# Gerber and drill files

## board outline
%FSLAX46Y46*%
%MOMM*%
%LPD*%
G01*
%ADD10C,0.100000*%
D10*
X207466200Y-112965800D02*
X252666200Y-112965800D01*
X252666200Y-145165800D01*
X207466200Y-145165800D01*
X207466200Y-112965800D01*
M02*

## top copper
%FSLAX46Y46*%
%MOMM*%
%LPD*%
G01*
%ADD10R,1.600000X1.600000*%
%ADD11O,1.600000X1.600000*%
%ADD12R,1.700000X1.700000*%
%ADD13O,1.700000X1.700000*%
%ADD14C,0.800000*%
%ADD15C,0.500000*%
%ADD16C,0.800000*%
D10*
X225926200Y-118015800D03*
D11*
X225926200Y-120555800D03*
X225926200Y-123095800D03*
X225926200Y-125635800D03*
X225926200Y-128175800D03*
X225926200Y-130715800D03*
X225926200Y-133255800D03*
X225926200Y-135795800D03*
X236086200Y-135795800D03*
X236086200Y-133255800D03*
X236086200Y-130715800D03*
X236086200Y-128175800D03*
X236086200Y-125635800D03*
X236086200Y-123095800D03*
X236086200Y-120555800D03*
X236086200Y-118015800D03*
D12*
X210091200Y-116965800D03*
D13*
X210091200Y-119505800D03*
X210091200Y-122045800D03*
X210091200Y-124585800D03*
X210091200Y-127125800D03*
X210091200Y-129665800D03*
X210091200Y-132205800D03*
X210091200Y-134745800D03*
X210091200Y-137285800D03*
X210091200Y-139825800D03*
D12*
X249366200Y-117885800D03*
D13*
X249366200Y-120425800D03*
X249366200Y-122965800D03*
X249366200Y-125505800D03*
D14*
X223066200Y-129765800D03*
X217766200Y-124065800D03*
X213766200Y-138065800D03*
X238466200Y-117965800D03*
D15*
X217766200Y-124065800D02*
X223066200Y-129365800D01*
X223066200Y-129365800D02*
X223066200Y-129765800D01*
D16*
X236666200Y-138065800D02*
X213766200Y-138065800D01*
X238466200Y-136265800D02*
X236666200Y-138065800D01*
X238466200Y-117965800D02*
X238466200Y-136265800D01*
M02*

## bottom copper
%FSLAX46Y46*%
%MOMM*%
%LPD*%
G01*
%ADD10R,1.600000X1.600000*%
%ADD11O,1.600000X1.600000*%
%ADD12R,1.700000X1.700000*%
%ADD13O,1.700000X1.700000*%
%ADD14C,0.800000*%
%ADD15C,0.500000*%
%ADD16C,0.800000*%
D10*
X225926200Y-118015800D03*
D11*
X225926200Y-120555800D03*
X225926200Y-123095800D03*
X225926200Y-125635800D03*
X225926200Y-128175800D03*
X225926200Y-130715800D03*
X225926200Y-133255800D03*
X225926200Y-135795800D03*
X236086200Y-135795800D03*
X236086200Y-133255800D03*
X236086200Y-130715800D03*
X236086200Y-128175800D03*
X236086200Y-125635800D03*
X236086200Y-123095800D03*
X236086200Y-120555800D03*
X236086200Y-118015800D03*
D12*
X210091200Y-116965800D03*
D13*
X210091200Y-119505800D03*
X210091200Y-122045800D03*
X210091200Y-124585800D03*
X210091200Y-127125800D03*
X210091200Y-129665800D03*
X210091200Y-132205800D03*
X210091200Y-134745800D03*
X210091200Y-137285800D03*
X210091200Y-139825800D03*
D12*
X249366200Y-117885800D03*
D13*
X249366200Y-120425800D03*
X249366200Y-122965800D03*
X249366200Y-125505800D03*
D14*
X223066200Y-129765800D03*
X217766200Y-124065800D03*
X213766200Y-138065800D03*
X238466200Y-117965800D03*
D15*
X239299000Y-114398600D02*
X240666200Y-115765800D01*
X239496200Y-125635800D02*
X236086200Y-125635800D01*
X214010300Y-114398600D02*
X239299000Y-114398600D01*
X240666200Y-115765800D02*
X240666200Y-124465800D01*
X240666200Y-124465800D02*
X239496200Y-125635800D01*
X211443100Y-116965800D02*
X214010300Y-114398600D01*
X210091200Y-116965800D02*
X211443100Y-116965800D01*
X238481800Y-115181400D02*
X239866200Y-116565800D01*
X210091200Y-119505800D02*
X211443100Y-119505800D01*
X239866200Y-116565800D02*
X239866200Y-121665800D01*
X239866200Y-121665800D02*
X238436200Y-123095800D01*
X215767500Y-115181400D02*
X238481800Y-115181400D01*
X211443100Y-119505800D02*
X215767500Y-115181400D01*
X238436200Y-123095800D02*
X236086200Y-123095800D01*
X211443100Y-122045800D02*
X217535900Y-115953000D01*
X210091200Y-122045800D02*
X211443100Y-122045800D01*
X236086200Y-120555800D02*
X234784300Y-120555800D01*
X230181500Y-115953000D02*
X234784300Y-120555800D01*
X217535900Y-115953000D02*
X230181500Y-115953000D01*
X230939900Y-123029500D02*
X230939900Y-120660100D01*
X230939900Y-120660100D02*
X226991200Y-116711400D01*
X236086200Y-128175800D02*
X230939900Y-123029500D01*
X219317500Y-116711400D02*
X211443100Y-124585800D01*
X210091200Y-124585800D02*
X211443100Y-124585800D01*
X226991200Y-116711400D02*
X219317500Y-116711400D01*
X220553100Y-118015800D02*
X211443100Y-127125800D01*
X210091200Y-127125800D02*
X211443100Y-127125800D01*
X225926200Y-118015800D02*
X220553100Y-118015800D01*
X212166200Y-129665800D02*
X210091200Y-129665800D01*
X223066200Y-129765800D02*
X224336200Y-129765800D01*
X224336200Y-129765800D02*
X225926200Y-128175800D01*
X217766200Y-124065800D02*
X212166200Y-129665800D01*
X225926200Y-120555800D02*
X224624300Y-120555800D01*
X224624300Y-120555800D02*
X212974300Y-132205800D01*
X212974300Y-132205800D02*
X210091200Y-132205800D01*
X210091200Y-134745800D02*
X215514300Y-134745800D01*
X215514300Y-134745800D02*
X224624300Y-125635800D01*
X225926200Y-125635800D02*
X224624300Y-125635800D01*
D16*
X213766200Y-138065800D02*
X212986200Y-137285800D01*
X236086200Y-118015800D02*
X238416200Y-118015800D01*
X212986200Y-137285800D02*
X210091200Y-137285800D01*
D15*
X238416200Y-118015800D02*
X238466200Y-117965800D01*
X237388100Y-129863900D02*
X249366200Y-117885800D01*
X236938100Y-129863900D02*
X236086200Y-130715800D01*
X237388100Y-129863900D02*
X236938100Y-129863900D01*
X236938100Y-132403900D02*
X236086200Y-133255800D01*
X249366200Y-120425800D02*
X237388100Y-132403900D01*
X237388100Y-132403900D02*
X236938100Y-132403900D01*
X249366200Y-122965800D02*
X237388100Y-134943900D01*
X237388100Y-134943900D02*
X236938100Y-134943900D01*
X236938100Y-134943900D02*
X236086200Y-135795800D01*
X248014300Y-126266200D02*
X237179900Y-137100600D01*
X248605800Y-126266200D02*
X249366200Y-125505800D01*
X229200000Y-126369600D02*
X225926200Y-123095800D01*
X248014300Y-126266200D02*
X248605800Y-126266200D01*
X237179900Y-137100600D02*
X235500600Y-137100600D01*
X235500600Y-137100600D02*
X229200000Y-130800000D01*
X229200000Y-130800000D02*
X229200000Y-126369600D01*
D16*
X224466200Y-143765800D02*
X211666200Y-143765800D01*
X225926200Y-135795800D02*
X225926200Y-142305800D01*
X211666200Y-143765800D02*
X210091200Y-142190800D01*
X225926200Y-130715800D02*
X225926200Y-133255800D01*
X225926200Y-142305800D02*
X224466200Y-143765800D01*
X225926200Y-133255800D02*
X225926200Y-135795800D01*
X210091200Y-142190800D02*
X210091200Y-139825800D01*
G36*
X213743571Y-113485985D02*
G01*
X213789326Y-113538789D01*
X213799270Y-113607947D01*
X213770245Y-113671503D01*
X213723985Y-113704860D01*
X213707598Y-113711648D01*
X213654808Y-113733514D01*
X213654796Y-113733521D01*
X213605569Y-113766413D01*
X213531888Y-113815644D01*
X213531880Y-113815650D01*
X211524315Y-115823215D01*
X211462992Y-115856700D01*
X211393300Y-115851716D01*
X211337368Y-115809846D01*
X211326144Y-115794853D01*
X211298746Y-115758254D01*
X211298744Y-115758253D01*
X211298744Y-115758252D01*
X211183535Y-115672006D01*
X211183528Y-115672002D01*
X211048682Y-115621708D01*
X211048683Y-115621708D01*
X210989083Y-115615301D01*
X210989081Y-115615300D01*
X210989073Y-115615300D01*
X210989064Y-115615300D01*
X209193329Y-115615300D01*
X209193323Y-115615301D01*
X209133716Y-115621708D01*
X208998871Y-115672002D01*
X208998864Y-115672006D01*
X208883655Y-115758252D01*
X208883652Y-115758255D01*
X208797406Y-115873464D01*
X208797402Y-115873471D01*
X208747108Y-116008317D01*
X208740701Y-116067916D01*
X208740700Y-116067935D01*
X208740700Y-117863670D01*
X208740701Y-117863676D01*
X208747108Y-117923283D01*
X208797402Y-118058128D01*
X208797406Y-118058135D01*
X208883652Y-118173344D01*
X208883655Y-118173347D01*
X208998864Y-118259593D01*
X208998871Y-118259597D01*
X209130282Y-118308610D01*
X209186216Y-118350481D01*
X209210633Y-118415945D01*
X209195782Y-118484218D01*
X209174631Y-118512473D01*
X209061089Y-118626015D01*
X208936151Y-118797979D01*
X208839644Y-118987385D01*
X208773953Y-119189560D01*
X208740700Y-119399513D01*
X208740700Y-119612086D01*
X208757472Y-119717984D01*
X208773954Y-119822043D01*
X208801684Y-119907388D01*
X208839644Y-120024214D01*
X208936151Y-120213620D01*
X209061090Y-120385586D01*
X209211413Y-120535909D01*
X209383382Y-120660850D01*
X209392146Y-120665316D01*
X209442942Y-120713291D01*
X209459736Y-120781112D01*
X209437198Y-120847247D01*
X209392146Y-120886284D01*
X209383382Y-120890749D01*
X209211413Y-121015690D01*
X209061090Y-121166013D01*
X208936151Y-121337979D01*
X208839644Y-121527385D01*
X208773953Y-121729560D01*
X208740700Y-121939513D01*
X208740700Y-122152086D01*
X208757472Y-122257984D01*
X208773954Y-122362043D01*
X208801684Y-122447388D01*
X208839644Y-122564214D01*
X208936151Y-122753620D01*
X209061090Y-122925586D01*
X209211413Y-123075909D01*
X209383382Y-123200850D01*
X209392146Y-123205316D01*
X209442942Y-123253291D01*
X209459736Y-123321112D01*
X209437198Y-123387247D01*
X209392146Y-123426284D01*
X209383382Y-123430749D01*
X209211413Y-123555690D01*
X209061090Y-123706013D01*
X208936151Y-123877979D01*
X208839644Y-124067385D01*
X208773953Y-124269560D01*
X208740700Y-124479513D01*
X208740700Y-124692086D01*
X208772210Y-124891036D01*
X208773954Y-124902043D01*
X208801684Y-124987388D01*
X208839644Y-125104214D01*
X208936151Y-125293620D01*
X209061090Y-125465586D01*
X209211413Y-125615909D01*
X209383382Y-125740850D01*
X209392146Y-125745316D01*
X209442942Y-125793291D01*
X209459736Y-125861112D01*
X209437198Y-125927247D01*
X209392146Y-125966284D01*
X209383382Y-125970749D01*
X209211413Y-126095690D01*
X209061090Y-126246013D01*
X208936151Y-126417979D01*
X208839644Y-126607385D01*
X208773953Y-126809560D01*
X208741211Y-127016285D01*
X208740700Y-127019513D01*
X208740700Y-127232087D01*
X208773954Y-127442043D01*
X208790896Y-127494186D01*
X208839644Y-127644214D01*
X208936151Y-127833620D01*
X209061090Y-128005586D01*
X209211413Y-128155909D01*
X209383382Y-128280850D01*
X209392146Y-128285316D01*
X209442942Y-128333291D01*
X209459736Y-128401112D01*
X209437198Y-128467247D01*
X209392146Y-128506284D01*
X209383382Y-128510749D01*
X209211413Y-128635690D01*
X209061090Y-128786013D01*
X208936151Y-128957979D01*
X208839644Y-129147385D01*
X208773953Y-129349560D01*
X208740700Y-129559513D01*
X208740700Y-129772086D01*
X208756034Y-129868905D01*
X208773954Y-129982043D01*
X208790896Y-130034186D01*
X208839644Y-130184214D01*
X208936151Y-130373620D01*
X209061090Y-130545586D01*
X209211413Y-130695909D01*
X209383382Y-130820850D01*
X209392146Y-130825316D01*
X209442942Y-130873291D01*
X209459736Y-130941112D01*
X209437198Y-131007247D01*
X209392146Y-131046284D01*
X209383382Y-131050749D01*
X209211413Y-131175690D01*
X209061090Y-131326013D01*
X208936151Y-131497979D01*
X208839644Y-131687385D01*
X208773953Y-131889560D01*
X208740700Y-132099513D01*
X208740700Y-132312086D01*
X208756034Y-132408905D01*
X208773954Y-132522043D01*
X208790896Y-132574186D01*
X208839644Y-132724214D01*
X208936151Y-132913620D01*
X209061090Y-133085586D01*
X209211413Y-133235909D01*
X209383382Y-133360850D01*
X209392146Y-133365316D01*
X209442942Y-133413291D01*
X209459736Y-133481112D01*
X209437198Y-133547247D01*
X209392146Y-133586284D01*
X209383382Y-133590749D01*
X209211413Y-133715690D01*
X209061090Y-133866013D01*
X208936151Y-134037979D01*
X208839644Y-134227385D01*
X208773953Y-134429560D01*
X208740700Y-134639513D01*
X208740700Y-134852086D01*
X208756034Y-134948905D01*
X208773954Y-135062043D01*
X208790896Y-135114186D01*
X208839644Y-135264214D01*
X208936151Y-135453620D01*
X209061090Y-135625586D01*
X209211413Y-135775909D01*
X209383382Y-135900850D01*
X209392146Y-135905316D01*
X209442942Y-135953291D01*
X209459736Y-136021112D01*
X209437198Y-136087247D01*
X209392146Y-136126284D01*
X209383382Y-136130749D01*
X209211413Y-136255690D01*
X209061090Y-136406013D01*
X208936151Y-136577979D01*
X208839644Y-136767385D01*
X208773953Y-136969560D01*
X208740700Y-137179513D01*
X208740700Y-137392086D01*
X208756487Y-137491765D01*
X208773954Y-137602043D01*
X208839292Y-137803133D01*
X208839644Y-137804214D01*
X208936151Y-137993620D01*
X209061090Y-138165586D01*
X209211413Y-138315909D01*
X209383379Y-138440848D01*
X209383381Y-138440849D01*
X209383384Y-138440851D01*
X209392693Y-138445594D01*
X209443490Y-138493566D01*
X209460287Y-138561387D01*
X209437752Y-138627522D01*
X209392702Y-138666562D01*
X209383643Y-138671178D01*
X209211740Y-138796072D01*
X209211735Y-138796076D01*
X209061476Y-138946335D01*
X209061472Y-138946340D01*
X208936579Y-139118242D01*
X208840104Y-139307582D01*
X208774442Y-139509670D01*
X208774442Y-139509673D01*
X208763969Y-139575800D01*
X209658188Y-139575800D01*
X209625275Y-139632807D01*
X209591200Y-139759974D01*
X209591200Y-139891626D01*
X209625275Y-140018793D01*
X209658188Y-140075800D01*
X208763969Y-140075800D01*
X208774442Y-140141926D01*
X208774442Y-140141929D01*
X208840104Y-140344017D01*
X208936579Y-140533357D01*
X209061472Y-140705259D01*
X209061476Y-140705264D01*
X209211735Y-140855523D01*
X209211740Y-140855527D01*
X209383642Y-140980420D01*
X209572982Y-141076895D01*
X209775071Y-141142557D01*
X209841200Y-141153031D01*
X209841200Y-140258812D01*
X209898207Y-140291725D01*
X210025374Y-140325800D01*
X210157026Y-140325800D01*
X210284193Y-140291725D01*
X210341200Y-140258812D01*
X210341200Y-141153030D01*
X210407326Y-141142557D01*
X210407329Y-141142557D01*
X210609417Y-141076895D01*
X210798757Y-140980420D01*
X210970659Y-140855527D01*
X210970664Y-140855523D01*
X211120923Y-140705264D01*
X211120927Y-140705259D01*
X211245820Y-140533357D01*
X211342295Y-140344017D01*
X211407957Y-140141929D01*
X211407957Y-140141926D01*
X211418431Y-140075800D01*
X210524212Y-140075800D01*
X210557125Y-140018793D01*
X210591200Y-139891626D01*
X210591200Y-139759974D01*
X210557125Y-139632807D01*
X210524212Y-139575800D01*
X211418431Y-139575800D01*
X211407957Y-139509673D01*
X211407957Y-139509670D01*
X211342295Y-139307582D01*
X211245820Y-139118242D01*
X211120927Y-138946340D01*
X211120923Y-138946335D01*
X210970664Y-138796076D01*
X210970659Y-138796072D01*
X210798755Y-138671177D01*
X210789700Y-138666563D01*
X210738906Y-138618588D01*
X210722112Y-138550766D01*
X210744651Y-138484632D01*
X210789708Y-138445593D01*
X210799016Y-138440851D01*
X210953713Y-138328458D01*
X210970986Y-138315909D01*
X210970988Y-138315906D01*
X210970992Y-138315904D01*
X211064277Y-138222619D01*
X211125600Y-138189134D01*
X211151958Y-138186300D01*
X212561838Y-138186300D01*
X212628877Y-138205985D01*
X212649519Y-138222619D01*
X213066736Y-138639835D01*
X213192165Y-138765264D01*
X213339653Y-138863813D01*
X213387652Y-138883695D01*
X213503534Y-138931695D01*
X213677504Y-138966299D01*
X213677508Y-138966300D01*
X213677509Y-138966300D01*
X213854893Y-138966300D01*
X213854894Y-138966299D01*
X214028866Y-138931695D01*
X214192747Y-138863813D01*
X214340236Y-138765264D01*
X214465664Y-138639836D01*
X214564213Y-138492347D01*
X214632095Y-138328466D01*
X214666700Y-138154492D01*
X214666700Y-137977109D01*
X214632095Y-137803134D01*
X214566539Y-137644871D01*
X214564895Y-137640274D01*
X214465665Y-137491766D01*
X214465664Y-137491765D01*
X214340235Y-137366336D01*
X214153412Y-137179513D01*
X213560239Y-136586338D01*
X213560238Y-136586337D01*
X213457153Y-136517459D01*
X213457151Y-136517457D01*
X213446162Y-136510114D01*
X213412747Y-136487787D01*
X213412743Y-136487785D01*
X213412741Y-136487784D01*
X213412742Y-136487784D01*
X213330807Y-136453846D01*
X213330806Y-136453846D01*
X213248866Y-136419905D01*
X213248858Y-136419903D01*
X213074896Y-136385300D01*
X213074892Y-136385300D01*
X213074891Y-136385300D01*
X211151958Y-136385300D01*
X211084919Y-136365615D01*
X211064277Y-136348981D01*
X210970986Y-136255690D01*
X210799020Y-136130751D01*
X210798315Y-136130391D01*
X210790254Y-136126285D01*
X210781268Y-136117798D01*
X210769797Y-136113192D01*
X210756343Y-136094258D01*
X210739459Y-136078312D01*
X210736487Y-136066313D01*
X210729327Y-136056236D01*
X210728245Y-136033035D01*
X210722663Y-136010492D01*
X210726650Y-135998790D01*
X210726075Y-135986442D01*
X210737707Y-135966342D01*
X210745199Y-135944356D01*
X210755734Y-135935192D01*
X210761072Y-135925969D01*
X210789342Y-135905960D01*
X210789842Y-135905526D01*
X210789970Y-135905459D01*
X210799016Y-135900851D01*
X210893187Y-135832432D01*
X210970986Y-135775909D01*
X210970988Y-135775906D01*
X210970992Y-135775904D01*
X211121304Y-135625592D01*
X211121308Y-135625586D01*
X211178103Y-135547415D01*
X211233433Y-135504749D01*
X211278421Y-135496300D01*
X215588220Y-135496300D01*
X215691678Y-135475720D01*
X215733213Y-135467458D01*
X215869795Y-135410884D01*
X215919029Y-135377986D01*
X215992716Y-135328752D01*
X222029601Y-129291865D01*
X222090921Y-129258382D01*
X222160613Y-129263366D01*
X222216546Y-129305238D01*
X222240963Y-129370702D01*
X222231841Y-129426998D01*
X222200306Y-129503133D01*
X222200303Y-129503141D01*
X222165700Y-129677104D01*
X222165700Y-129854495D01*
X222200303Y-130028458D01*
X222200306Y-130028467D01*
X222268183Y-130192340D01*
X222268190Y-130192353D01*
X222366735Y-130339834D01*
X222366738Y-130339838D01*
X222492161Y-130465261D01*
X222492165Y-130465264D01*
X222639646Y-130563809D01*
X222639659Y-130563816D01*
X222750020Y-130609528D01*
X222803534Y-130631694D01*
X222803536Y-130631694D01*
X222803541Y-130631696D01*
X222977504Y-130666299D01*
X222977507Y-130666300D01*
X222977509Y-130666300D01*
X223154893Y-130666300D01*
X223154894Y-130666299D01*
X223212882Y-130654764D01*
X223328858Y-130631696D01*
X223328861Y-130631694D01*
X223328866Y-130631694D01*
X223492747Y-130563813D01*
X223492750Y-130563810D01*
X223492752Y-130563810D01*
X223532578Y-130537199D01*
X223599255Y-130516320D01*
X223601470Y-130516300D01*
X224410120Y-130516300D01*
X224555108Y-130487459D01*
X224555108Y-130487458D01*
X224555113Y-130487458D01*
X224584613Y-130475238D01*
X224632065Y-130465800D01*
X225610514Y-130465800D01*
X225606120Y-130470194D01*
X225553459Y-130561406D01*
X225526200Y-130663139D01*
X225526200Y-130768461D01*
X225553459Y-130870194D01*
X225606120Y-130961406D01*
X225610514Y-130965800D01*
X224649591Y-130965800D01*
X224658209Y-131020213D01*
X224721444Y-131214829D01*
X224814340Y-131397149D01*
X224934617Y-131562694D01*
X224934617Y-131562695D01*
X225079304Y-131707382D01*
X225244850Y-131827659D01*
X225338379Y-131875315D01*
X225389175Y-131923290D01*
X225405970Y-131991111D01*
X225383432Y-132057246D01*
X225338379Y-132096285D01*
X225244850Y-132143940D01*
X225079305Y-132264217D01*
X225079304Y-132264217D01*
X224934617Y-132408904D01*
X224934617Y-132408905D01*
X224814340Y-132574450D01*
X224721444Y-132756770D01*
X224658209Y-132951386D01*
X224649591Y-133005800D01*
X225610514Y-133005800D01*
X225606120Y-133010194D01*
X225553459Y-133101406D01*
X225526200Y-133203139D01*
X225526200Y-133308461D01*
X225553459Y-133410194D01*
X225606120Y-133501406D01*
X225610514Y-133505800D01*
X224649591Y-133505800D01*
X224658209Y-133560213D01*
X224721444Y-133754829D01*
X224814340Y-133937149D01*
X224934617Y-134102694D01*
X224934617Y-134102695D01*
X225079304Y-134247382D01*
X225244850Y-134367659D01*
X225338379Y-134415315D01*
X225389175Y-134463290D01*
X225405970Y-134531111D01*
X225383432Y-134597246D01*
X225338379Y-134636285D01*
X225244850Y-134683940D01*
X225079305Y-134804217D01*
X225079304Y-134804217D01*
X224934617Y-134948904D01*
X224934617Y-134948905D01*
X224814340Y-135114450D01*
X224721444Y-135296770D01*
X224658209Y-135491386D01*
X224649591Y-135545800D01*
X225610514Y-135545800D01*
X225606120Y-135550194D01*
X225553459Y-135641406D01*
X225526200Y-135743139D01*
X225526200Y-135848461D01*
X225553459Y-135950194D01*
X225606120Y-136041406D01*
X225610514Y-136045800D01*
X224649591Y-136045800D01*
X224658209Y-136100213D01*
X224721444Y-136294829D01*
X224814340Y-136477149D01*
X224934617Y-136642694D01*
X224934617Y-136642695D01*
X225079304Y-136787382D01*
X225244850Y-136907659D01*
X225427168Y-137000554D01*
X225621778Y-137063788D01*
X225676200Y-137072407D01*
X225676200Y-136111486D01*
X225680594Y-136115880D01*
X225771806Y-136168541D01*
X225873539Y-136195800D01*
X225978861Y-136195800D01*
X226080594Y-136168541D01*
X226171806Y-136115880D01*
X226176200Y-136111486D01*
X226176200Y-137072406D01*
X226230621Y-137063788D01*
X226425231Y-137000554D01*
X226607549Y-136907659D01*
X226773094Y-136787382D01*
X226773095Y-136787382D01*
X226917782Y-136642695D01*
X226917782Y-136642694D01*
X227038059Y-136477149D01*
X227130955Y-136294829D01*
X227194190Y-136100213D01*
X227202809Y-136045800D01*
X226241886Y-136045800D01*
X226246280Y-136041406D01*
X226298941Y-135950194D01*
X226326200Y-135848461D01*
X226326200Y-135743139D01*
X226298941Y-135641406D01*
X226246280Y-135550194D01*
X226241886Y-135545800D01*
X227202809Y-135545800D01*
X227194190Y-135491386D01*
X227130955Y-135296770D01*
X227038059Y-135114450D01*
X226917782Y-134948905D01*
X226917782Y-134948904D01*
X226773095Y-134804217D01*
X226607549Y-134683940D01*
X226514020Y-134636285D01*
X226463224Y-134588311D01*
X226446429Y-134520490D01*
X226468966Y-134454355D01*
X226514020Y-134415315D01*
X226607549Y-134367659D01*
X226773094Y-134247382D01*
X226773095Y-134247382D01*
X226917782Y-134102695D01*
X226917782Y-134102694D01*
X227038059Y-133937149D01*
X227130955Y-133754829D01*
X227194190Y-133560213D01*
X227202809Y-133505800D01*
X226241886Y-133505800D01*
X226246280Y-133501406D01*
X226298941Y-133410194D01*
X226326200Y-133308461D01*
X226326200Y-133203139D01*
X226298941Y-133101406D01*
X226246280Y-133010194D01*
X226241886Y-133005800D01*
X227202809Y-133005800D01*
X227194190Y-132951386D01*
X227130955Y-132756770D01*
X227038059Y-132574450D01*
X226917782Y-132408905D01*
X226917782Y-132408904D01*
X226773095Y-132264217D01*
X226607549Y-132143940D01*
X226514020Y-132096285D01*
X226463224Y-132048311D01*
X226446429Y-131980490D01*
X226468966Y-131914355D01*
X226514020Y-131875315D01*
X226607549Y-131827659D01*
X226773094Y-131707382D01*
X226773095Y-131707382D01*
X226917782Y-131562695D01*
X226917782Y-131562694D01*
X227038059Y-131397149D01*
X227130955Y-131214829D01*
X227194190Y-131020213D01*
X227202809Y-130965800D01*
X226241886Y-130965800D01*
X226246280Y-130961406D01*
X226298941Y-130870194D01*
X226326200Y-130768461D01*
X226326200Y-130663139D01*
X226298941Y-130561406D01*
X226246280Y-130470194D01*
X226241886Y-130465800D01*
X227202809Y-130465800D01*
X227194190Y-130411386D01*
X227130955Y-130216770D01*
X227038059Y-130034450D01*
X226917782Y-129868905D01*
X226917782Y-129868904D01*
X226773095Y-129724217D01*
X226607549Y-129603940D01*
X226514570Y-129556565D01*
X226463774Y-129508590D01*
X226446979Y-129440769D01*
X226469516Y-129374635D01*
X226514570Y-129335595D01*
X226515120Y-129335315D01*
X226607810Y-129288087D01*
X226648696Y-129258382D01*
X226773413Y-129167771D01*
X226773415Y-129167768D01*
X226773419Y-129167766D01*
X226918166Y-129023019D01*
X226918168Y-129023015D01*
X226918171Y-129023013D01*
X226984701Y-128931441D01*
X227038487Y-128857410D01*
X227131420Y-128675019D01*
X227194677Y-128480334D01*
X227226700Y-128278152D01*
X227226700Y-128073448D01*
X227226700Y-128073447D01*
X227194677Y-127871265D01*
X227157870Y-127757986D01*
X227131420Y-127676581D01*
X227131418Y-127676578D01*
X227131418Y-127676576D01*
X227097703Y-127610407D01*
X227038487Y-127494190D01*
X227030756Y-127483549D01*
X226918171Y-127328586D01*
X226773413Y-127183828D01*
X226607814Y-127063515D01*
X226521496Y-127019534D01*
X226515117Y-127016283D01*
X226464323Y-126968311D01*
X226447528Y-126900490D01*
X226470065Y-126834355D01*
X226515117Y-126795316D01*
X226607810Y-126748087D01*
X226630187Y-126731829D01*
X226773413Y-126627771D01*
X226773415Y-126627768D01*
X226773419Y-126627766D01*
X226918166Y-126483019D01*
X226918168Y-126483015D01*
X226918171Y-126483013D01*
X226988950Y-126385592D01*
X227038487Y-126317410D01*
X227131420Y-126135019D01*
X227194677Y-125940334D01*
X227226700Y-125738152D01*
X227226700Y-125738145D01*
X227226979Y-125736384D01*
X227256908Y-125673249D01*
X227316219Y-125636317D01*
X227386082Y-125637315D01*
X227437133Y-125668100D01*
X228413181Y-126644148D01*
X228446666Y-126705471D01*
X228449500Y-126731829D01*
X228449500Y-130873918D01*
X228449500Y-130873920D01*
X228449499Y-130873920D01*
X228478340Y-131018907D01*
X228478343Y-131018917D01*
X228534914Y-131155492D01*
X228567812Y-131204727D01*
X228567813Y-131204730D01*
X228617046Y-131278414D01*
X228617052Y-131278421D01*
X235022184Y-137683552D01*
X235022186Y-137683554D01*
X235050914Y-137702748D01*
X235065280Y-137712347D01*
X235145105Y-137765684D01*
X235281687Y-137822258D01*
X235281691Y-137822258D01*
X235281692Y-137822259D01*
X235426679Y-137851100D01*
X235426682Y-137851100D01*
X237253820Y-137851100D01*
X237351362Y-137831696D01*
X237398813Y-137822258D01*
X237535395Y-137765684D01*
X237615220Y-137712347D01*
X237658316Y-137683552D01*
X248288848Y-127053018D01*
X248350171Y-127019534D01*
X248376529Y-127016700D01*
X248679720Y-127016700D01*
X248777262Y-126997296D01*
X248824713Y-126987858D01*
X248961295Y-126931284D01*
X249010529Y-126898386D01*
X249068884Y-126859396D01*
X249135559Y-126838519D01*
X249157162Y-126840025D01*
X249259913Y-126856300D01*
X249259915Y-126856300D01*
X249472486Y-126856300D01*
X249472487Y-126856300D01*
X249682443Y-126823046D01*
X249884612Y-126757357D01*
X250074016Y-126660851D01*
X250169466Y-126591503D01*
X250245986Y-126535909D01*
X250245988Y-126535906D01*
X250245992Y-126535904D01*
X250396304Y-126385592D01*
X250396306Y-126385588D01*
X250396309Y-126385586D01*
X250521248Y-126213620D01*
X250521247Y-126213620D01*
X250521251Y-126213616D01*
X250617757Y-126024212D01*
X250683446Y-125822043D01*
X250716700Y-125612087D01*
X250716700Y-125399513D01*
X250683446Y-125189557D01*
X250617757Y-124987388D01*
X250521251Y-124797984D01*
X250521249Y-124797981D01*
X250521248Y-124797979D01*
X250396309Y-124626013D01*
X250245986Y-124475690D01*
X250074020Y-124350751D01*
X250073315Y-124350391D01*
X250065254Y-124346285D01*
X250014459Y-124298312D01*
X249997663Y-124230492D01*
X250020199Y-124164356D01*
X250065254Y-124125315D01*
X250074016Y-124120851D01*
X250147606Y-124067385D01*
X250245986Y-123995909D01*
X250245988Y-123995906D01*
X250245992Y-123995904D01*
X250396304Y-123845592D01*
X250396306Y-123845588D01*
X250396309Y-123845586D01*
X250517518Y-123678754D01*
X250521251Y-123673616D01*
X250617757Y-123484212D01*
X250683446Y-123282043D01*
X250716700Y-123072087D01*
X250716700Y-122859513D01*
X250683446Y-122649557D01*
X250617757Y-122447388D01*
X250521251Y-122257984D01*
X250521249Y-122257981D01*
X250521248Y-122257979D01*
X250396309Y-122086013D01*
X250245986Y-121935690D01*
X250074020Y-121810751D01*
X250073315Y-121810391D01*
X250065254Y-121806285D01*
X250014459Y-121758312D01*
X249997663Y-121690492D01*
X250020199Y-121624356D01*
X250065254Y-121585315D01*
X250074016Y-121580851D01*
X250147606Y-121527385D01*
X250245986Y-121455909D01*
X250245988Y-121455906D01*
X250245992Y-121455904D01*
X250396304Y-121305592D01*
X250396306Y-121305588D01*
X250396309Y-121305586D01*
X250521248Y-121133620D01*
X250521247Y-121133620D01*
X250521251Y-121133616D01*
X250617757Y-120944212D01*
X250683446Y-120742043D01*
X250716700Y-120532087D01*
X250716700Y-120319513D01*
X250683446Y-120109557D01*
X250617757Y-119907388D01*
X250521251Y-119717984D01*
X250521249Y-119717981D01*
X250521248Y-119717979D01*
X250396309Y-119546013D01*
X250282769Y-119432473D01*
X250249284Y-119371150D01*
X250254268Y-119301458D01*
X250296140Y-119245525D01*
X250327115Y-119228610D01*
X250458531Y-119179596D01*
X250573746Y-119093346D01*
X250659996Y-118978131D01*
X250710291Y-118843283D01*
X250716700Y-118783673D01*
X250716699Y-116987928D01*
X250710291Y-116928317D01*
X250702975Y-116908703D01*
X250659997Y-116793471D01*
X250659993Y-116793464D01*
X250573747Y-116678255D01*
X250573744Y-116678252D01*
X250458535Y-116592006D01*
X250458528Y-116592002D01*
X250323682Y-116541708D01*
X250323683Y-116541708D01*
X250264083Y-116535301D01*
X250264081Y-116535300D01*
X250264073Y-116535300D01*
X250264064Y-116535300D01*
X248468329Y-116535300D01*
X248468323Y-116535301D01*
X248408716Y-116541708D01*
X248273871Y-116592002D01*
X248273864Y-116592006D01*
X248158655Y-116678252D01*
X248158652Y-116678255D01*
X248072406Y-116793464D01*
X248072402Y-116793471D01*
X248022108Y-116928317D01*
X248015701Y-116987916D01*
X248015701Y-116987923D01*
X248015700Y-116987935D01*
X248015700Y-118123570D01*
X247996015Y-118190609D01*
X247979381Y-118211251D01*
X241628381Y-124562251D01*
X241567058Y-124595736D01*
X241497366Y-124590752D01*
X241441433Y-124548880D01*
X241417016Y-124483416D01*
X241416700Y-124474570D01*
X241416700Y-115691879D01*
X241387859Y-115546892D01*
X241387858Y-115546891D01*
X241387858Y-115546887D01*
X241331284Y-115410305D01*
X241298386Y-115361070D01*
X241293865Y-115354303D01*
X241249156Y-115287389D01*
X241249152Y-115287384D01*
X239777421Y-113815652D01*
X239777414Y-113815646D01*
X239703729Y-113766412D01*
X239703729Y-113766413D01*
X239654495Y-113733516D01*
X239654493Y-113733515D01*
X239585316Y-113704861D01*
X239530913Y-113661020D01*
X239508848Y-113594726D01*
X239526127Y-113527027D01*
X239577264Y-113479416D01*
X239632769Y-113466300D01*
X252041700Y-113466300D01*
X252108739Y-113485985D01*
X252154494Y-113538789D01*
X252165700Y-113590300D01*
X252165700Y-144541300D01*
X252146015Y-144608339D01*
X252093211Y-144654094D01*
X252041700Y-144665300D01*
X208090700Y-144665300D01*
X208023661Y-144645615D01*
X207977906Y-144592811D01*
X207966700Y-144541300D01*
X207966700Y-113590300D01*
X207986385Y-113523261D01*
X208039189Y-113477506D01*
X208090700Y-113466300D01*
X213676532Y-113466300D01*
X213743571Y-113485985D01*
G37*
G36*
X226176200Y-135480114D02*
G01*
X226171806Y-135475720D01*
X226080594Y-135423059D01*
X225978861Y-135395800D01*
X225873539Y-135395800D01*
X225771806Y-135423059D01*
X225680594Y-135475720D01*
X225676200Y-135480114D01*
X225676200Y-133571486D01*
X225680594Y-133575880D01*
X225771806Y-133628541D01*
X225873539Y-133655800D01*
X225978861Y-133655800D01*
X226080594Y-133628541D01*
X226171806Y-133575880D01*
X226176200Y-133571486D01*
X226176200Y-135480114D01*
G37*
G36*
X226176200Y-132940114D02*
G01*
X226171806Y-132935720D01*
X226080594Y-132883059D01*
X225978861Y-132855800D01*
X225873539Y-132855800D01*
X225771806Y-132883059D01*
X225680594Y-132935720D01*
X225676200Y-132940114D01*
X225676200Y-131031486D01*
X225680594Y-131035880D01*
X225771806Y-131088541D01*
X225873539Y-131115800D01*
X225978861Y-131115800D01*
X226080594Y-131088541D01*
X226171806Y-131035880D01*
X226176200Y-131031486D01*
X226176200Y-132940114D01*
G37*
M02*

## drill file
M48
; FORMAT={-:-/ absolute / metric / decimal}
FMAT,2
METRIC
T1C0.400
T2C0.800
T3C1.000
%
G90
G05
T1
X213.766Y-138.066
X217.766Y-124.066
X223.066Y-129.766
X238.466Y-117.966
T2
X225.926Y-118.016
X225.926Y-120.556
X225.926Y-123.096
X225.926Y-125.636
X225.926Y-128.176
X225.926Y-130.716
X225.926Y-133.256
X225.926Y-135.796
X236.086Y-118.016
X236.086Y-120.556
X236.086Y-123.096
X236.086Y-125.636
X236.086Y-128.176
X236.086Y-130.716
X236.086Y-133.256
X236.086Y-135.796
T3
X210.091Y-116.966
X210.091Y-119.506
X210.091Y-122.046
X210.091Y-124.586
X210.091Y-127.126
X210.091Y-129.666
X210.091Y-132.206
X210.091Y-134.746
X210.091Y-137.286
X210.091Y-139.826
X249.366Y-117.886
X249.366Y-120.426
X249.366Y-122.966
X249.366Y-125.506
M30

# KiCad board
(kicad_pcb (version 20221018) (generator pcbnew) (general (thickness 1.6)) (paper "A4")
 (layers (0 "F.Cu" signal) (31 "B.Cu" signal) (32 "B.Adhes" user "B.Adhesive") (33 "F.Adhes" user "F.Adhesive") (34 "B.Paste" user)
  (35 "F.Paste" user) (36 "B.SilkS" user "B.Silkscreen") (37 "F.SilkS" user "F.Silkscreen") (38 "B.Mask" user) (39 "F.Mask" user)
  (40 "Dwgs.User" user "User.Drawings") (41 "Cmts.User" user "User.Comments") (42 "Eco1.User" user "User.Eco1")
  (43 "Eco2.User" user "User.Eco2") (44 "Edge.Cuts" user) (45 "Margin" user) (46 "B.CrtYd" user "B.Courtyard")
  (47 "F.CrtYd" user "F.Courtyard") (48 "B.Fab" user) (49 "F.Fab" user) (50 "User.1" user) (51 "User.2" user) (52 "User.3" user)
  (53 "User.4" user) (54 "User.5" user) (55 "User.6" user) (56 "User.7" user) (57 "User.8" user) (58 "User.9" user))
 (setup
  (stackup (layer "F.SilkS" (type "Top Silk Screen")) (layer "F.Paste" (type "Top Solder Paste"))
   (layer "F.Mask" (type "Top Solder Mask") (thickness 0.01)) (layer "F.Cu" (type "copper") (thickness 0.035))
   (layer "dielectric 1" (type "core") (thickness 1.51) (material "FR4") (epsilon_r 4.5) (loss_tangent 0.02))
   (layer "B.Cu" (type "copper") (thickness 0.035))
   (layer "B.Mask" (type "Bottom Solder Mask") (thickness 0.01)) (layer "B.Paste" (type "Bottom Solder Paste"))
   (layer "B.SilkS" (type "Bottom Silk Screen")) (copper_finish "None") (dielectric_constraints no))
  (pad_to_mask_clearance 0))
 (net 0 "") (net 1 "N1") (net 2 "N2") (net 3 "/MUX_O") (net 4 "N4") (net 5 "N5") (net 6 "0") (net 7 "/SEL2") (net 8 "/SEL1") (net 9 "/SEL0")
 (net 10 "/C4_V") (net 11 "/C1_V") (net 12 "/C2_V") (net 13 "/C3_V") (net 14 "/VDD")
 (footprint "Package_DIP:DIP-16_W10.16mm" (layer "F.Cu") (at 225.9262 118.0158)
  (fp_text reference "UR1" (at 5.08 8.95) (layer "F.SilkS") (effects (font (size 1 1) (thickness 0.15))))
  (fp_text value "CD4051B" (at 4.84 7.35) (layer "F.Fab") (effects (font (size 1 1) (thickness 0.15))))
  (pad "1" thru_hole rect (at 0 0) (size 1.6 1.6) (drill 0.8) (layers "*.Cu" "*.Mask") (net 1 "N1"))
  (pad "2" thru_hole oval (at 0 2.54) (size 1.6 1.6) (drill 0.8) (layers "*.Cu" "*.Mask") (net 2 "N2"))
  (pad "3" thru_hole oval (at 0 5.08) (size 1.6 1.6) (drill 0.8) (layers "*.Cu" "*.Mask") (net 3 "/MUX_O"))
  (pad "4" thru_hole oval (at 0 7.62) (size 1.6 1.6) (drill 0.8) (layers "*.Cu" "*.Mask") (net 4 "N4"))
  (pad "5" thru_hole oval (at 0 10.16) (size 1.6 1.6) (drill 0.8) (layers "*.Cu" "*.Mask") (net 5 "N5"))
  (pad "6" thru_hole oval (at 0 12.7) (size 1.6 1.6) (drill 0.8) (layers "*.Cu" "*.Mask") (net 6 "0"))
  (pad "7" thru_hole oval (at 0 15.24) (size 1.6 1.6) (drill 0.8) (layers "*.Cu" "*.Mask") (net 6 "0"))
  (pad "8" thru_hole oval (at 0 17.78) (size 1.6 1.6) (drill 0.8) (layers "*.Cu" "*.Mask") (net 6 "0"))
  (pad "9" thru_hole oval (at 10.16 17.78) (size 1.6 1.6) (drill 0.8) (layers "*.Cu" "*.Mask") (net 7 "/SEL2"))
  (pad "10" thru_hole oval (at 10.16 15.24) (size 1.6 1.6) (drill 0.8) (layers "*.Cu" "*.Mask") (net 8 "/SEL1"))
  (pad "11" thru_hole oval (at 10.16 12.7) (size 1.6 1.6) (drill 0.8) (layers "*.Cu" "*.Mask") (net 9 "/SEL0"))
  (pad "12" thru_hole oval (at 10.16 10.16) (size 1.6 1.6) (drill 0.8) (layers "*.Cu" "*.Mask") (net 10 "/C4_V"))
  (pad "13" thru_hole oval (at 10.16 7.62) (size 1.6 1.6) (drill 0.8) (layers "*.Cu" "*.Mask") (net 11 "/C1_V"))
  (pad "14" thru_hole oval (at 10.16 5.08) (size 1.6 1.6) (drill 0.8) (layers "*.Cu" "*.Mask") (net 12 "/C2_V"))
  (pad "15" thru_hole oval (at 10.16 2.54) (size 1.6 1.6) (drill 0.8) (layers "*.Cu" "*.Mask") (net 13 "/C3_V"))
  (pad "16" thru_hole oval (at 10.16 0) (size 1.6 1.6) (drill 0.8) (layers "*.Cu" "*.Mask") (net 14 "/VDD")))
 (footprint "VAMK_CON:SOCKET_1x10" (layer "F.Cu") (at 210.0912 116.9658)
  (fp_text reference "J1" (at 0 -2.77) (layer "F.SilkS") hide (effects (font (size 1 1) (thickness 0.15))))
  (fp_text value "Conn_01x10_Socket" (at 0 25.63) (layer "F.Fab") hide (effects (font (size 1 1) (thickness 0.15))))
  (pad "1" thru_hole rect (at 0 0) (size 1.7 1.7) (drill 1) (layers "*.Cu" "*.Mask") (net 11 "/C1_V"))
  (pad "2" thru_hole oval (at 0 2.54) (size 1.7 1.7) (drill 1) (layers "*.Cu" "*.Mask") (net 12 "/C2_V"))
  (pad "3" thru_hole oval (at 0 5.08) (size 1.7 1.7) (drill 1) (layers "*.Cu" "*.Mask") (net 13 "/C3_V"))
  (pad "4" thru_hole oval (at 0 7.62) (size 1.7 1.7) (drill 1) (layers "*.Cu" "*.Mask") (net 10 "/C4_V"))
  (pad "5" thru_hole oval (at 0 10.16) (size 1.7 1.7) (drill 1) (layers "*.Cu" "*.Mask") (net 1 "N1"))
  (pad "6" thru_hole oval (at 0 12.7) (size 1.7 1.7) (drill 1) (layers "*.Cu" "*.Mask") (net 5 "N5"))
  (pad "7" thru_hole oval (at 0 15.24) (size 1.7 1.7) (drill 1) (layers "*.Cu" "*.Mask") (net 2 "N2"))
  (pad "8" thru_hole oval (at 0 17.78) (size 1.7 1.7) (drill 1) (layers "*.Cu" "*.Mask") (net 4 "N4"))
  (pad "9" thru_hole oval (at 0 20.32) (size 1.7 1.7) (drill 1) (layers "*.Cu" "*.Mask") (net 14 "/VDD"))
  (pad "10" thru_hole oval (at 0 22.86) (size 1.7 1.7) (drill 1) (layers "*.Cu" "*.Mask") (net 6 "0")))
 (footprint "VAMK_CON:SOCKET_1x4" (layer "F.Cu") (at 249.3662 117.8858)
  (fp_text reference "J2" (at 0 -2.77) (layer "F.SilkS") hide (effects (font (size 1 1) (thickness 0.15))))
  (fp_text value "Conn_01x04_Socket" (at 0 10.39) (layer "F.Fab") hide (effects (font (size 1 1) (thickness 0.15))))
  (pad "1" thru_hole rect (at 0 0) (size 1.7 1.7) (drill 1) (layers "*.Cu" "*.Mask") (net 9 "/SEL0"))
  (pad "2" thru_hole oval (at 0 2.54) (size 1.7 1.7) (drill 1) (layers "*.Cu" "*.Mask") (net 8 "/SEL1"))
  (pad "3" thru_hole oval (at 0 5.08) (size 1.7 1.7) (drill 1) (layers "*.Cu" "*.Mask") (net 7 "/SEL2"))
  (pad "4" thru_hole oval (at 0 7.62) (size 1.7 1.7) (drill 1) (layers "*.Cu" "*.Mask") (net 3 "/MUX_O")))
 (gr_rect (start 207.4662 112.9658) (end 252.6662 145.1658) (stroke (width 0.1) (type default)) (fill none) (layer "Edge.Cuts"))
 (segment (start 239.299 114.3986) (end 240.6662 115.7658) (width 0.5) (layer "B.Cu") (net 11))
 (segment (start 239.4962 125.6358) (end 236.0862 125.6358) (width 0.5) (layer "B.Cu") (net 11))
 (segment (start 214.0103 114.3986) (end 239.299 114.3986) (width 0.5) (layer "B.Cu") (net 11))
 (segment (start 240.6662 115.7658) (end 240.6662 124.4658) (width 0.5) (layer "B.Cu") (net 11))
 (segment (start 240.6662 124.4658) (end 239.4962 125.6358) (width 0.5) (layer "B.Cu") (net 11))
 (segment (start 211.4431 116.9658) (end 214.0103 114.3986) (width 0.5) (layer "B.Cu") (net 11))
 (segment (start 210.0912 116.9658) (end 211.4431 116.9658) (width 0.5) (layer "B.Cu") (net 11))
 (segment (start 238.4818 115.1814) (end 239.8662 116.5658) (width 0.5) (layer "B.Cu") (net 12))
 (segment (start 210.0912 119.5058) (end 211.4431 119.5058) (width 0.5) (layer "B.Cu") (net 12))
 (segment (start 239.8662 116.5658) (end 239.8662 121.6658) (width 0.5) (layer "B.Cu") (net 12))
 (segment (start 239.8662 121.6658) (end 238.4362 123.0958) (width 0.5) (layer "B.Cu") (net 12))
 (segment (start 215.7675 115.1814) (end 238.4818 115.1814) (width 0.5) (layer "B.Cu") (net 12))
 (segment (start 211.4431 119.5058) (end 215.7675 115.1814) (width 0.5) (layer "B.Cu") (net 12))
 (segment (start 238.4362 123.0958) (end 236.0862 123.0958) (width 0.5) (layer "B.Cu") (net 12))
 (segment (start 211.4431 122.0458) (end 217.5359 115.953) (width 0.5) (layer "B.Cu") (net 13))
 (segment (start 210.0912 122.0458) (end 211.4431 122.0458) (width 0.5) (layer "B.Cu") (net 13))
 (segment (start 236.0862 120.5558) (end 234.7843 120.5558) (width 0.5) (layer "B.Cu") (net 13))
 (segment (start 230.1815 115.953) (end 234.7843 120.5558) (width 0.5) (layer "B.Cu") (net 13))
 (segment (start 217.5359 115.953) (end 230.1815 115.953) (width 0.5) (layer "B.Cu") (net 13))
 (segment (start 230.9399 123.0295) (end 230.9399 120.6601) (width 0.5) (layer "B.Cu") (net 10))
 (segment (start 230.9399 120.6601) (end 226.9912 116.7114) (width 0.5) (layer "B.Cu") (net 10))
 (segment (start 236.0862 128.1758) (end 230.9399 123.0295) (width 0.5) (layer "B.Cu") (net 10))
 (segment (start 219.3175 116.7114) (end 211.4431 124.5858) (width 0.5) (layer "B.Cu") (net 10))
 (segment (start 210.0912 124.5858) (end 211.4431 124.5858) (width 0.5) (layer "B.Cu") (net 10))
 (segment (start 226.9912 116.7114) (end 219.3175 116.7114) (width 0.5) (layer "B.Cu") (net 10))
 (segment (start 220.5531 118.0158) (end 211.4431 127.1258) (width 0.5) (layer "B.Cu") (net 1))
 (segment (start 210.0912 127.1258) (end 211.4431 127.1258) (width 0.5) (layer "B.Cu") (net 1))
 (segment (start 225.9262 118.0158) (end 220.5531 118.0158) (width 0.5) (layer "B.Cu") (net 1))
 (segment (start 217.7662 124.0658) (end 223.0662 129.3658) (width 0.5) (layer "F.Cu") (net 5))
 (segment (start 223.0662 129.3658) (end 223.0662 129.7658) (width 0.5) (layer "F.Cu") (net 5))
 (via (at 223.0662 129.7658) (size 0.8) (drill 0.4) (layers "F.Cu" "B.Cu") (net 5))
 (via (at 217.7662 124.0658) (size 0.8) (drill 0.4) (layers "F.Cu" "B.Cu") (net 5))
 (segment (start 212.1662 129.6658) (end 210.0912 129.6658) (width 0.5) (layer "B.Cu") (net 5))
 (segment (start 223.0662 129.7658) (end 224.3362 129.7658) (width 0.5) (layer "B.Cu") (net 5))
 (segment (start 224.3362 129.7658) (end 225.9262 128.1758) (width 0.5) (layer "B.Cu") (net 5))
 (segment (start 217.7662 124.0658) (end 212.1662 129.6658) (width 0.5) (layer "B.Cu") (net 5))
 (segment (start 225.9262 120.5558) (end 224.6243 120.5558) (width 0.5) (layer "B.Cu") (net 2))
 (segment (start 224.6243 120.5558) (end 212.9743 132.2058) (width 0.5) (layer "B.Cu") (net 2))
 (segment (start 212.9743 132.2058) (end 210.0912 132.2058) (width 0.5) (layer "B.Cu") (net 2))
 (segment (start 210.0912 134.7458) (end 215.5143 134.7458) (width 0.5) (layer "B.Cu") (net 4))
 (segment (start 215.5143 134.7458) (end 224.6243 125.6358) (width 0.5) (layer "B.Cu") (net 4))
 (segment (start 225.9262 125.6358) (end 224.6243 125.6358) (width 0.5) (layer "B.Cu") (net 4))
 (segment (start 236.6662 138.0658) (end 213.7662 138.0658) (width 0.8) (layer "F.Cu") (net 14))
 (segment (start 238.4662 136.2658) (end 236.6662 138.0658) (width 0.8) (layer "F.Cu") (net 14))
 (segment (start 238.4662 117.9658) (end 238.4662 136.2658) (width 0.8) (layer "F.Cu") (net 14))
 (via (at 213.7662 138.0658) (size 0.8) (drill 0.4) (layers "F.Cu" "B.Cu") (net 14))
 (via (at 238.4662 117.9658) (size 0.8) (drill 0.4) (layers "F.Cu" "B.Cu") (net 14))
 (segment (start 213.7662 138.0658) (end 212.9862 137.2858) (width 0.8) (layer "B.Cu") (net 14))
 (segment (start 236.0862 118.0158) (end 238.4162 118.0158) (width 0.8) (layer "B.Cu") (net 14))
 (segment (start 212.9862 137.2858) (end 210.0912 137.2858) (width 0.8) (layer "B.Cu") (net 14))
 (segment (start 238.4162 118.0158) (end 238.4662 117.9658) (width 0.5) (layer "B.Cu") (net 14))
 (segment (start 237.3881 129.8639) (end 249.3662 117.8858) (width 0.5) (layer "B.Cu") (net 9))
 (segment (start 236.9381 129.8639) (end 236.0862 130.7158) (width 0.5) (layer "B.Cu") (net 9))
 (segment (start 237.3881 129.8639) (end 236.9381 129.8639) (width 0.5) (layer "B.Cu") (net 9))
 (segment (start 236.9381 132.4039) (end 236.0862 133.2558) (width 0.5) (layer "B.Cu") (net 8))
 (segment (start 249.3662 120.4258) (end 237.3881 132.4039) (width 0.5) (layer "B.Cu") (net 8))
 (segment (start 237.3881 132.4039) (end 236.9381 132.4039) (width 0.5) (layer "B.Cu") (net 8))
 (segment (start 249.3662 122.9658) (end 237.3881 134.9439) (width 0.5) (layer "B.Cu") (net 7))
 (segment (start 237.3881 134.9439) (end 236.9381 134.9439) (width 0.5) (layer "B.Cu") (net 7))
 (segment (start 236.9381 134.9439) (end 236.0862 135.7958) (width 0.5) (layer "B.Cu") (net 7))
 (segment (start 248.0143 126.2662) (end 237.1799 137.1006) (width 0.5) (layer "B.Cu") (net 3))
 (segment (start 248.6058 126.2662) (end 249.3662 125.5058) (width 0.5) (layer "B.Cu") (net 3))
 (segment (start 229.2 126.3696) (end 225.9262 123.0958) (width 0.5) (layer "B.Cu") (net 3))
 (segment (start 248.0143 126.2662) (end 248.6058 126.2662) (width 0.5) (layer "B.Cu") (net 3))
 (segment (start 237.1799 137.1006) (end 235.5006 137.1006) (width 0.5) (layer "B.Cu") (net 3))
 (segment (start 235.5006 137.1006) (end 229.2 130.8) (width 0.5) (layer "B.Cu") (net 3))
 (segment (start 229.2 130.8) (end 229.2 126.3696) (width 0.5) (layer "B.Cu") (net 3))
 (segment (start 224.4662 143.7658) (end 211.6662 143.7658) (width 0.8) (layer "B.Cu") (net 6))
 (segment (start 225.9262 135.7958) (end 225.9262 142.3058) (width 0.8) (layer "B.Cu") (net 6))
 (segment (start 211.6662 143.7658) (end 210.0912 142.1908) (width 0.8) (layer "B.Cu") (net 6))
 (segment (start 225.9262 130.7158) (end 225.9262 133.2558) (width 0.8) (layer "B.Cu") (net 6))
 (segment (start 225.9262 142.3058) (end 224.4662 143.7658) (width 0.8) (layer "B.Cu") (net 6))
 (segment (start 225.9262 133.2558) (end 225.9262 135.7958) (width 0.8) (layer "B.Cu") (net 6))
 (segment (start 210.0912 142.1908) (end 210.0912 139.8258) (width 0.8) (layer "B.Cu") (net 6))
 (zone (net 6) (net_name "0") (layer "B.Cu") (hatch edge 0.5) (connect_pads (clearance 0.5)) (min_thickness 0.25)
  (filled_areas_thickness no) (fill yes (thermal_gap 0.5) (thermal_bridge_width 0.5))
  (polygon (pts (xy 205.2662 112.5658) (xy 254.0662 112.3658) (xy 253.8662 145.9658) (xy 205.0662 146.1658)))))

